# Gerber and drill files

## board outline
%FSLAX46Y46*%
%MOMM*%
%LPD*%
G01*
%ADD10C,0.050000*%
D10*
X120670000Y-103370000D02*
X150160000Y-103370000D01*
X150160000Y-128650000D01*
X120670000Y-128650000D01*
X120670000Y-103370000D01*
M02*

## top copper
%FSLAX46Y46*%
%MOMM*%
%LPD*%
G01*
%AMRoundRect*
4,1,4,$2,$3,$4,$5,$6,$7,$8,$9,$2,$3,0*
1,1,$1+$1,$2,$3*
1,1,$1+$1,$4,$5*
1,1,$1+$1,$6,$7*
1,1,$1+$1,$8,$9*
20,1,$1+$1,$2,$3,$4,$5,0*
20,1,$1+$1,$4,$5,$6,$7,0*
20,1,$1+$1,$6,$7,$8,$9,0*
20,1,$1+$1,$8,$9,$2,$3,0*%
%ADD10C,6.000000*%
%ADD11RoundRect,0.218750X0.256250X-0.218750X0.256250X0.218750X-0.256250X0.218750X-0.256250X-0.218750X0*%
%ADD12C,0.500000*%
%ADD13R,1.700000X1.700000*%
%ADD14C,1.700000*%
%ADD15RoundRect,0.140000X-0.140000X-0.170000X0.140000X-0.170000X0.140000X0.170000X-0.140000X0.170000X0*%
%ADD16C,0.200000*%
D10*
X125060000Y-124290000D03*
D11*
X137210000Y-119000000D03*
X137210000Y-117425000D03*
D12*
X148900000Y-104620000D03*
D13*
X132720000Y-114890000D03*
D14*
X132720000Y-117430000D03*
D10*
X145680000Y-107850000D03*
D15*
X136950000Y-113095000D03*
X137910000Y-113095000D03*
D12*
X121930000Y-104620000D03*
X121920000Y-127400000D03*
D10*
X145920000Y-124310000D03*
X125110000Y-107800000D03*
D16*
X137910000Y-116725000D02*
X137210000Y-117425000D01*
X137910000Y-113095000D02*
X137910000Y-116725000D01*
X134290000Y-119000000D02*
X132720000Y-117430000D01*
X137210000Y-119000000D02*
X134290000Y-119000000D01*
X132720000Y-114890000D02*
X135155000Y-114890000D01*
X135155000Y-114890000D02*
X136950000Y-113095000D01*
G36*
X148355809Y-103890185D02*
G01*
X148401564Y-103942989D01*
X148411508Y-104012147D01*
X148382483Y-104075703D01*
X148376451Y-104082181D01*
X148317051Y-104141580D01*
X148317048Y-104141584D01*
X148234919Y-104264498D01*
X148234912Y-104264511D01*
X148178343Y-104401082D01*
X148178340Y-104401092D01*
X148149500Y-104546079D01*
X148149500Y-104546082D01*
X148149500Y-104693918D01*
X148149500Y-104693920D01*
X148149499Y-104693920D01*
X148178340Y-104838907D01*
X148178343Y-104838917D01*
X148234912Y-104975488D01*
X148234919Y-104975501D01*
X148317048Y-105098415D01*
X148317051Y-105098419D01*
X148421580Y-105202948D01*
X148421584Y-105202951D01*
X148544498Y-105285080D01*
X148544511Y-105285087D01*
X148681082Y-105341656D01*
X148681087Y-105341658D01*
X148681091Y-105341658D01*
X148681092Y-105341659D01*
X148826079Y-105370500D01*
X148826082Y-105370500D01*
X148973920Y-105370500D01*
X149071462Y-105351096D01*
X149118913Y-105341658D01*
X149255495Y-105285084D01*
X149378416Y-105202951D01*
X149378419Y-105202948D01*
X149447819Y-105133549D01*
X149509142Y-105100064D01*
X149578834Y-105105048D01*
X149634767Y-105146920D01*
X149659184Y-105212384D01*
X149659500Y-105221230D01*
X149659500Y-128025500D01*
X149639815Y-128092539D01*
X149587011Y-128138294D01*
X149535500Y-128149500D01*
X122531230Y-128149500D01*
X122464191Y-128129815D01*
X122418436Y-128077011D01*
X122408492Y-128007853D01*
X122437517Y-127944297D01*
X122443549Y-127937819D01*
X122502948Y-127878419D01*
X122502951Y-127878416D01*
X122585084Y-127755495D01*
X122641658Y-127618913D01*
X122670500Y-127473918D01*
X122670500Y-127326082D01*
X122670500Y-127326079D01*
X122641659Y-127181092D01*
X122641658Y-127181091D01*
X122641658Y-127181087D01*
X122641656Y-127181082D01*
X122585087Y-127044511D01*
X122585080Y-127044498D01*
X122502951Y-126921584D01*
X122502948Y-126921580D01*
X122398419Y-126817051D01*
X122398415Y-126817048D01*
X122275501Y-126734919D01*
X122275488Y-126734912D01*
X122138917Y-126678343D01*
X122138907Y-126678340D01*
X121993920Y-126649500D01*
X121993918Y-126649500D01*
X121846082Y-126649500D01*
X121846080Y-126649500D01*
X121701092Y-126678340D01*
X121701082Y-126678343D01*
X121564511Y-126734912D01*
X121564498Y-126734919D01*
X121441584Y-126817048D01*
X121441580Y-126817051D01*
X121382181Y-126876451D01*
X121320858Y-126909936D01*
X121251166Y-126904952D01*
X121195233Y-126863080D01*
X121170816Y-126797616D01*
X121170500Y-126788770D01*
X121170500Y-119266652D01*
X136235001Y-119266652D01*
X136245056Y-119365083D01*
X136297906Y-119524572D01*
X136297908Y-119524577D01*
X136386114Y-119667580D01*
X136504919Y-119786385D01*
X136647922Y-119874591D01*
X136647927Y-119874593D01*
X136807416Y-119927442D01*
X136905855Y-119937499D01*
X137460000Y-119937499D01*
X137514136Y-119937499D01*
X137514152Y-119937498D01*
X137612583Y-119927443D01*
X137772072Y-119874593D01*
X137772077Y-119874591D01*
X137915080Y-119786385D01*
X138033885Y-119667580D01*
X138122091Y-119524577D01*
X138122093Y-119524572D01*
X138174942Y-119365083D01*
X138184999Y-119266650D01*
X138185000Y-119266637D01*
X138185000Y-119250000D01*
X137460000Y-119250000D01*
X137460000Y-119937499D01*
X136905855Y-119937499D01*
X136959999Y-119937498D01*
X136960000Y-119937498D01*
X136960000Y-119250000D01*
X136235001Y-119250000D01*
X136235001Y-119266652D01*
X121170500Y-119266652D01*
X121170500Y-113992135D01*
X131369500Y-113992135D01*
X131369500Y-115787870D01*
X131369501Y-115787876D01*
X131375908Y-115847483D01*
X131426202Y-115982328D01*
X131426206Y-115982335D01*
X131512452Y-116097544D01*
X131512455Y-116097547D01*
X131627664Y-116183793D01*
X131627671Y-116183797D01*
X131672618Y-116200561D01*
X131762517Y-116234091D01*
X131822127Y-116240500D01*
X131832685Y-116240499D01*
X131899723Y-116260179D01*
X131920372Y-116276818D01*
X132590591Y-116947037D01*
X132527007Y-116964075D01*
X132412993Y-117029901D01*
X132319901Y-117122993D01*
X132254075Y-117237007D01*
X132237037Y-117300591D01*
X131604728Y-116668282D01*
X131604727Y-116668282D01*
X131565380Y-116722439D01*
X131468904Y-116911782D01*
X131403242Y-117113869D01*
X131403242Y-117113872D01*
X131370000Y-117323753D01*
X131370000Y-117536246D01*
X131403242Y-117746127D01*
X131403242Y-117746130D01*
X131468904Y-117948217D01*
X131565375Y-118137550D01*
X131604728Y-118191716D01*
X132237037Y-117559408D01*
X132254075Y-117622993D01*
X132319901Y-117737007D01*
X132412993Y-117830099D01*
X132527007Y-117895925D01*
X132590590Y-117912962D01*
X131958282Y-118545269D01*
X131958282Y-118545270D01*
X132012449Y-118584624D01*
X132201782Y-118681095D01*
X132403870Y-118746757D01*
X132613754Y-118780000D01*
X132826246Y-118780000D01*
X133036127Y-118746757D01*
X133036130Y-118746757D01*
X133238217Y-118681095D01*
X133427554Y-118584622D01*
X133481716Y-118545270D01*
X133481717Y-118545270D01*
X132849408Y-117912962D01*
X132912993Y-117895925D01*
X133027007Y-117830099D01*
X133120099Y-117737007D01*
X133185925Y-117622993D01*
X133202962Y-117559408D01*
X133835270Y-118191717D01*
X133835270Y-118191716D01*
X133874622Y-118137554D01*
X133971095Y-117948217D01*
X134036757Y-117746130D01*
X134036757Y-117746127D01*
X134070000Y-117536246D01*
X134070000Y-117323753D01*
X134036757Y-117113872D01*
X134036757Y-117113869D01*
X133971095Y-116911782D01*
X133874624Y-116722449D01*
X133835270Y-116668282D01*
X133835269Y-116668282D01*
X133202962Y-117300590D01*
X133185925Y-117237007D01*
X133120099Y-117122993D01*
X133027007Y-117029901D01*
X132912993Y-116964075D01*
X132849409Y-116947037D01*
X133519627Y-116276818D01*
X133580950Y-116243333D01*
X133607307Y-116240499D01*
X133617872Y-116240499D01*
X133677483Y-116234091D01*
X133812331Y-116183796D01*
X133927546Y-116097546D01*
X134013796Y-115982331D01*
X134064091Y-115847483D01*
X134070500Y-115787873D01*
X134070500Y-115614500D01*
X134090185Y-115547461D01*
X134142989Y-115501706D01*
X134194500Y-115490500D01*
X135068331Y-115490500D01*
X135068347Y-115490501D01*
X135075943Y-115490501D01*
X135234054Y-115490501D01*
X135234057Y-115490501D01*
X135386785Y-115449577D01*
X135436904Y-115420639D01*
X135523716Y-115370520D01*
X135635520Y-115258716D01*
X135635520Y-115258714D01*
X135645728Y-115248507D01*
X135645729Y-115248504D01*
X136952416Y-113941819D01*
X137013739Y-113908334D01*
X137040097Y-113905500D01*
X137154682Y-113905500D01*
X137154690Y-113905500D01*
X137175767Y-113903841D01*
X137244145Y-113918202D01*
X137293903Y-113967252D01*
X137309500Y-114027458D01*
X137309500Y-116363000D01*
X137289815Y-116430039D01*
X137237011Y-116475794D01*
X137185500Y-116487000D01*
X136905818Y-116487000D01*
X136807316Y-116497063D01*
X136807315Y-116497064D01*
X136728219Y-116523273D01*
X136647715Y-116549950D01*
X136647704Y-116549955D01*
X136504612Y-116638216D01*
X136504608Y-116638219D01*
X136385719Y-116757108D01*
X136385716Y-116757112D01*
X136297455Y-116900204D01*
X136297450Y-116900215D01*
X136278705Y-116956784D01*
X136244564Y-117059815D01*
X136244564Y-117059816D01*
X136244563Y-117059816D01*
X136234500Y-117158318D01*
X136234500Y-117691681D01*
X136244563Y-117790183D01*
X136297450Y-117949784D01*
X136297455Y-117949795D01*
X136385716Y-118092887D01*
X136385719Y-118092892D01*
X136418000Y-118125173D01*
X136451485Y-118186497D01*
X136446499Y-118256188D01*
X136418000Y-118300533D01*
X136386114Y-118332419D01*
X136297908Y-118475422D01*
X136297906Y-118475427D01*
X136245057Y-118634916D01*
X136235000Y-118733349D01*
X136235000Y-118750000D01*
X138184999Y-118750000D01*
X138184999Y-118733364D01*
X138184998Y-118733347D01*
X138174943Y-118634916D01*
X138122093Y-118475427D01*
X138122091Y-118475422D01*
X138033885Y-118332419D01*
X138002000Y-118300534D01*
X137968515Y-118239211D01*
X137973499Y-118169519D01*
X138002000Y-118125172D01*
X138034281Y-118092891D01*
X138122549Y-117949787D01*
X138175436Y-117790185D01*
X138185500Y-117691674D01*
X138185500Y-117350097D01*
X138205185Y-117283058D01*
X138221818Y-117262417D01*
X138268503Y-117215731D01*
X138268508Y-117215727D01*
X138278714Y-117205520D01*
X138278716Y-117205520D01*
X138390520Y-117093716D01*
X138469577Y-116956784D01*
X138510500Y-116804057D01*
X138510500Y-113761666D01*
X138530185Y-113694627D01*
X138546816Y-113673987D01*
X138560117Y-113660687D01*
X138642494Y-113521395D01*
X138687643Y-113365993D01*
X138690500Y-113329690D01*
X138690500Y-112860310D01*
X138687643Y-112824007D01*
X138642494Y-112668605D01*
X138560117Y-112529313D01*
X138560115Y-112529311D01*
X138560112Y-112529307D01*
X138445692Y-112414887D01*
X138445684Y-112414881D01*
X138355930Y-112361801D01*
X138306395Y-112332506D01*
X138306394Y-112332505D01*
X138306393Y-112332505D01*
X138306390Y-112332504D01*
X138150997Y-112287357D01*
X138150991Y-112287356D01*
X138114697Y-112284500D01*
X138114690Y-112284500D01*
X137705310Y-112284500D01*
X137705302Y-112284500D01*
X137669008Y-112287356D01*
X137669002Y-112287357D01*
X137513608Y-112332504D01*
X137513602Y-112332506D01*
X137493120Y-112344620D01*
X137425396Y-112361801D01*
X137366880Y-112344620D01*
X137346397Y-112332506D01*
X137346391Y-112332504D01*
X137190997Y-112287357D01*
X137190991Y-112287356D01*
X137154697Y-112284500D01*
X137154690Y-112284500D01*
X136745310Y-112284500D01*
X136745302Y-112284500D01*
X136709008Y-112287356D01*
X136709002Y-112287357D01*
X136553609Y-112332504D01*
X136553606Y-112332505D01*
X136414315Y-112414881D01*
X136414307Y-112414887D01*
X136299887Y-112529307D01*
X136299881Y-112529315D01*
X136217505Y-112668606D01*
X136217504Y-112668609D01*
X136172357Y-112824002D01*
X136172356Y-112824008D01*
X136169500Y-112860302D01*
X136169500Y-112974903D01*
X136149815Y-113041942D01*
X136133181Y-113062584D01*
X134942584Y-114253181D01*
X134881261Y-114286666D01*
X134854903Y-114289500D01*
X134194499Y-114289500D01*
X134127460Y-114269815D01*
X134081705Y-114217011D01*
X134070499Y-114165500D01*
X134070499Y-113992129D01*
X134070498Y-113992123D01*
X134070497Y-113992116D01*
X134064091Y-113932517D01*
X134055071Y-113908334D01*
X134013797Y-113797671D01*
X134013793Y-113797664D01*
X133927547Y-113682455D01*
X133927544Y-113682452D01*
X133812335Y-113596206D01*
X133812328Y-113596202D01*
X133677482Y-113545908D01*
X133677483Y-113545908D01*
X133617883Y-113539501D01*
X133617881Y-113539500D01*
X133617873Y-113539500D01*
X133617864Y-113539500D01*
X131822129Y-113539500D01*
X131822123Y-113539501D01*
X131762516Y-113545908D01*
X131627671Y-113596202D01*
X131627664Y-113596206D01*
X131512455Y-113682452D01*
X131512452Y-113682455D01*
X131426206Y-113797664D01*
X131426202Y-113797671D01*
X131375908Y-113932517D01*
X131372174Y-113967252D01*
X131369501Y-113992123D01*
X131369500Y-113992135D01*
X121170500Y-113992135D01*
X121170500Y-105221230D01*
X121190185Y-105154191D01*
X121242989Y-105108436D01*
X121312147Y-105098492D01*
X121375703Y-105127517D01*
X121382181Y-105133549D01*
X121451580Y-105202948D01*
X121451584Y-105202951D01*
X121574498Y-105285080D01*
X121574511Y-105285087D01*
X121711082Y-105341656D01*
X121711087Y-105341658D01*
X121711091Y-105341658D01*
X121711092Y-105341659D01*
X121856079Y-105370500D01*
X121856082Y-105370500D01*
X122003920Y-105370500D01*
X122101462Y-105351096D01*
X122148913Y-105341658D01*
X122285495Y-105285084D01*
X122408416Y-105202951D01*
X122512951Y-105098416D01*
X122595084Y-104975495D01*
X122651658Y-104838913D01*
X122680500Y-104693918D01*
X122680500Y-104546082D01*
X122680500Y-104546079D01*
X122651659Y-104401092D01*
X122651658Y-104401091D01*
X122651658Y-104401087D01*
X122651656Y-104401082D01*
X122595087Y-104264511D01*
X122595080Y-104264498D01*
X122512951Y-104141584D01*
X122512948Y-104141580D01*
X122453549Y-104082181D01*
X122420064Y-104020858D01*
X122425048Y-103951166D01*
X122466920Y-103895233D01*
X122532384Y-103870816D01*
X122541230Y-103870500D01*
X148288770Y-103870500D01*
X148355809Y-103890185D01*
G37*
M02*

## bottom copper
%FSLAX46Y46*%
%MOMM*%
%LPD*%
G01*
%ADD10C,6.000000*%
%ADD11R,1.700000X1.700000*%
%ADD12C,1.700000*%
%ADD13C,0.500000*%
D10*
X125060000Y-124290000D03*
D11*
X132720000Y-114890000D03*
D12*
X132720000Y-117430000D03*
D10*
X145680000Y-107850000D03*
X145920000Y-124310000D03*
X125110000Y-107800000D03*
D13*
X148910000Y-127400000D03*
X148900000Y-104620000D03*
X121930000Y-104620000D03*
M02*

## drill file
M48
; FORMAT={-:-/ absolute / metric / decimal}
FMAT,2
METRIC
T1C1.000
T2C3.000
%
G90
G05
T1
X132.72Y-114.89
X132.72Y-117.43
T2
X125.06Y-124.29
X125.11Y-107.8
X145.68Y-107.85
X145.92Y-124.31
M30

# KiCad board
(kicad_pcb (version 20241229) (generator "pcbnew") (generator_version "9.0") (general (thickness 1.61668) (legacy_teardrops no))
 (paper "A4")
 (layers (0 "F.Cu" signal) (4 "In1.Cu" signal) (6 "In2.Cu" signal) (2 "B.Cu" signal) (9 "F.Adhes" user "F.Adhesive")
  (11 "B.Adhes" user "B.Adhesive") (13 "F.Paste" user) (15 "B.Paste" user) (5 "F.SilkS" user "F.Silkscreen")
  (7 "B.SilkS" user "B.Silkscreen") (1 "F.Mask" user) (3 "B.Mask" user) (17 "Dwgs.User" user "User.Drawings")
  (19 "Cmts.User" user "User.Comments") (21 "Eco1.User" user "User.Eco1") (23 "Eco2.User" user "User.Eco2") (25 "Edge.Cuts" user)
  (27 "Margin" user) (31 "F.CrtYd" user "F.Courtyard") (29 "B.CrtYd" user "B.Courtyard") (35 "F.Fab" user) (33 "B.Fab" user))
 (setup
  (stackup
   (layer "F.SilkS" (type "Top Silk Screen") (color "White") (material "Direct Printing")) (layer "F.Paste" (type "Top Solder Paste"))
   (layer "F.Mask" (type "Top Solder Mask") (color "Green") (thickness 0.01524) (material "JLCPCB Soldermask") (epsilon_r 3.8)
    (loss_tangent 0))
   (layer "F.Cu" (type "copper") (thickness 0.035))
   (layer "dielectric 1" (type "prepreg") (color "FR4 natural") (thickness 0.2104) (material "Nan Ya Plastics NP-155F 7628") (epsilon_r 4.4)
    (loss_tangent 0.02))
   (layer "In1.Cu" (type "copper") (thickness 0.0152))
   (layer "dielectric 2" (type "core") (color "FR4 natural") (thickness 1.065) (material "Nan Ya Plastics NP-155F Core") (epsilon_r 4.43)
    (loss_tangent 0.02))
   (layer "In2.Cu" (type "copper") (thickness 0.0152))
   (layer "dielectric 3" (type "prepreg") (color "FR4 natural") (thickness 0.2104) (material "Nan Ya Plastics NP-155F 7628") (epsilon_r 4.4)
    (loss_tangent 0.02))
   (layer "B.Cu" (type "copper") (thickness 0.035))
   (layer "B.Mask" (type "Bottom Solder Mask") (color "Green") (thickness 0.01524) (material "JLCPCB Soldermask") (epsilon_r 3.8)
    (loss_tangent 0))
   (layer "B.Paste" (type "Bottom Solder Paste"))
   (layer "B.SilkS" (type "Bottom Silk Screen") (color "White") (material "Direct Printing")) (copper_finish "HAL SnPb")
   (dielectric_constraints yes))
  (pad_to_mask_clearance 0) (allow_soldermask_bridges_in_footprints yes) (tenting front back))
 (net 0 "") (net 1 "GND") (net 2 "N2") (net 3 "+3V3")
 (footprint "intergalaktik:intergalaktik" (layer "F.Cu") (at 135.4 104.33)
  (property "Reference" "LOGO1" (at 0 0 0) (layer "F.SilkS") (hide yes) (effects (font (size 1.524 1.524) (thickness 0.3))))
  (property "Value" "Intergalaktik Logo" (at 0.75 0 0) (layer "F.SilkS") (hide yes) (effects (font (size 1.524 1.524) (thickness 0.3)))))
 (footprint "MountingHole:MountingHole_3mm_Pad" (layer "F.Cu") (at 125.06 124.29)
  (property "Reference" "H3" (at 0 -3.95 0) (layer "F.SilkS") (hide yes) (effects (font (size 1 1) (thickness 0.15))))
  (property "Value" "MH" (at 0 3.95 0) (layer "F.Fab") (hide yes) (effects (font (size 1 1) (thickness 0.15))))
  (pad "1" thru_hole circle (at 0 0) (size 6 6) (drill 3) (layers "*.Cu" "*.Mask") (remove_unused_layers no) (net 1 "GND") (zone_connect 2)))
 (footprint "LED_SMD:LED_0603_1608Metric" (layer "F.Cu") (at 137.21 118.2125 90)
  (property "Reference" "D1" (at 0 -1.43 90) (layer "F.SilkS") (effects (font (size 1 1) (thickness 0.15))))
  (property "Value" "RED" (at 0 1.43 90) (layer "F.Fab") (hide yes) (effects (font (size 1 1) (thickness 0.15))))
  (pad "1" smd roundrect (at -0.7875 0 90) (size 0.875 0.95) (layers "F.Cu" "F.Mask" "F.Paste") (roundrect_rratio 0.25) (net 1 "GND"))
  (pad "2" smd roundrect (at 0.7875 0 90) (size 0.875 0.95) (layers "F.Cu" "F.Mask" "F.Paste") (roundrect_rratio 0.25) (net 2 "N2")))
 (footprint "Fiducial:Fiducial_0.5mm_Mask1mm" (layer "F.Cu") (at 148.9 104.62)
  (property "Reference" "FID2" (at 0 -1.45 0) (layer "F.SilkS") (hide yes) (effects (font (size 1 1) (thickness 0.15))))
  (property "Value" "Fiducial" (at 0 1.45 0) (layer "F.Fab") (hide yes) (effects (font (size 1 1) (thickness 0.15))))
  (pad "" smd circle (at 0 0) (size 0.5 0.5) (layers "F.Cu" "F.Mask") (solder_mask_margin 0.25)))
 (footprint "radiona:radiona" (layer "F.Cu") (at 135.68 125.26)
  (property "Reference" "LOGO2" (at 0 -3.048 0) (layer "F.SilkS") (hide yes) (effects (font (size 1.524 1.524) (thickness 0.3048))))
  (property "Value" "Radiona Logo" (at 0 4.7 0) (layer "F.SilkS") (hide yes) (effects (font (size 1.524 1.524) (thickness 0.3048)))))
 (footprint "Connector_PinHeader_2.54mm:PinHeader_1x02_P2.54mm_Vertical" (layer "F.Cu") (at 132.72 114.89)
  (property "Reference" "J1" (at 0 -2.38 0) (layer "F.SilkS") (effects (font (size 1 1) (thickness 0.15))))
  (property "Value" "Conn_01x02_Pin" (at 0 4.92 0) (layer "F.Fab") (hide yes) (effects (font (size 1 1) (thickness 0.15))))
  (pad "1" thru_hole rect (at 0 0) (size 1.7 1.7) (drill 1) (layers "*.Cu" "*.Mask") (remove_unused_layers no) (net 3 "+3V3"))
  (pad "2" thru_hole circle (at 0 2.54) (size 1.7 1.7) (drill 1) (layers "*.Cu" "*.Mask") (remove_unused_layers no) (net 1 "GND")))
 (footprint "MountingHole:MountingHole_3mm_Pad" (layer "F.Cu") (at 145.68 107.85)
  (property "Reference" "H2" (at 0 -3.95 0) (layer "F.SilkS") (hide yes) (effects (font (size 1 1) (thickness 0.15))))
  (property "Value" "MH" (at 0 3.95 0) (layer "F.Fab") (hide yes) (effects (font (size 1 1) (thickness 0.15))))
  (pad "1" thru_hole circle (at 0 0) (size 6 6) (drill 3) (layers "*.Cu" "*.Mask") (remove_unused_layers no) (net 1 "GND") (zone_connect 2)))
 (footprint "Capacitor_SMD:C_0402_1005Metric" (layer "F.Cu") (at 137.43 113.095)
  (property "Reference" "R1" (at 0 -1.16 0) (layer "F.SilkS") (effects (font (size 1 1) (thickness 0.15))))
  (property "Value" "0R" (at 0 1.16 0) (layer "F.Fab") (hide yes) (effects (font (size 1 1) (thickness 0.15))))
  (pad "1" smd roundrect (at -0.48 0) (size 0.56 0.62) (layers "F.Cu" "F.Mask" "F.Paste") (roundrect_rratio 0.25) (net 3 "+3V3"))
  (pad "2" smd roundrect (at 0.48 0) (size 0.56 0.62) (layers "F.Cu" "F.Mask" "F.Paste") (roundrect_rratio 0.25) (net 2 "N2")))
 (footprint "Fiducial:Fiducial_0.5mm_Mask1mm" (layer "F.Cu") (at 121.93 104.62)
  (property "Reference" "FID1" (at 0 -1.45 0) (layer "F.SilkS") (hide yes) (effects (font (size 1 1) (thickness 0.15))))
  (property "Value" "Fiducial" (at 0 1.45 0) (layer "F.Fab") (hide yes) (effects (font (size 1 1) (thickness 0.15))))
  (pad "" smd circle (at 0 0) (size 0.5 0.5) (layers "F.Cu" "F.Mask") (solder_mask_margin 0.25)))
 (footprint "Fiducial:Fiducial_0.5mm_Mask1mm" (layer "F.Cu") (at 121.92 127.4)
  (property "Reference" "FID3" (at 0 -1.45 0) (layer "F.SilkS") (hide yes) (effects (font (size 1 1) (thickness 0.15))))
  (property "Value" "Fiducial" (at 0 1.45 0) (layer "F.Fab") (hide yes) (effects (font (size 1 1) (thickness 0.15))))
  (pad "" smd circle (at 0 0) (size 0.5 0.5) (layers "F.Cu" "F.Mask") (solder_mask_margin 0.25)))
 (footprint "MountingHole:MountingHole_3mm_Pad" (layer "F.Cu") (at 145.92 124.31)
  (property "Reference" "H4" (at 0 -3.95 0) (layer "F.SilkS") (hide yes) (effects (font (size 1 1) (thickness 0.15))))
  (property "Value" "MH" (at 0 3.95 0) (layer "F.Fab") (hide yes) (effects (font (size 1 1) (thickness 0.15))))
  (pad "1" thru_hole circle (at 0 0) (size 6 6) (drill 3) (layers "*.Cu" "*.Mask") (remove_unused_layers no) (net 1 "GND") (zone_connect 2)))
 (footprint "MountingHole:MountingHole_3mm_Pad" (layer "F.Cu") (at 125.11 107.8)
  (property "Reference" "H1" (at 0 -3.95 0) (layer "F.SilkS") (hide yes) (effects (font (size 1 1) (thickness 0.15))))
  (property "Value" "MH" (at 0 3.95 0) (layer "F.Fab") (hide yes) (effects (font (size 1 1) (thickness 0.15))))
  (pad "1" thru_hole circle (at 0 0) (size 6 6) (drill 3) (layers "*.Cu" "*.Mask") (remove_unused_layers no) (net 1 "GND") (zone_connect 2)))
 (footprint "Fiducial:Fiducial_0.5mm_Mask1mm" (layer "B.Cu") (at 148.91 127.4)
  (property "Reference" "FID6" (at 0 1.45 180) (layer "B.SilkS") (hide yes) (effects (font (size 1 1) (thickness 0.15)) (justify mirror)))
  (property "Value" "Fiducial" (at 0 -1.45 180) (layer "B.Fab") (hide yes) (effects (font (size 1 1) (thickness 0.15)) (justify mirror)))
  (pad "" smd circle (at 0 0) (size 0.5 0.5) (layers "B.Cu" "B.Mask") (solder_mask_margin 0.25)))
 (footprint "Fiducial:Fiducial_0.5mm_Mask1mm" (layer "B.Cu") (at 148.9 104.62)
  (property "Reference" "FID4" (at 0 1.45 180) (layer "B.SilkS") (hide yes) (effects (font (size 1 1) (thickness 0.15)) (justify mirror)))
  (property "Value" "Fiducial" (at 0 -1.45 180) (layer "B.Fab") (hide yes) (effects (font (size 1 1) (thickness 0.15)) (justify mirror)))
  (pad "" smd circle (at 0 0) (size 0.5 0.5) (layers "B.Cu" "B.Mask") (solder_mask_margin 0.25)))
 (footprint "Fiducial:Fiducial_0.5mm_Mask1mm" (layer "B.Cu") (at 121.93 104.62)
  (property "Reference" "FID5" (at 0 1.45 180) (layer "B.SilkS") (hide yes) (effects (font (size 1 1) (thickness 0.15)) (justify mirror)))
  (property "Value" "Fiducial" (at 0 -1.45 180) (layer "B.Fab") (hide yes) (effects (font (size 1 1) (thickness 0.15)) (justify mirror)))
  (pad "" smd circle (at 0 0) (size 0.5 0.5) (layers "B.Cu" "B.Mask") (solder_mask_margin 0.25)))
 (gr_rect (start 120.67 103.37) (end 150.16 128.65) (stroke (width 0.05) (type default)) (fill no) (layer "Edge.Cuts"))
 (segment (start 137.91 116.725) (end 137.21 117.425) (width 0.2) (layer "F.Cu") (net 2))
 (segment (start 137.91 113.095) (end 137.91 116.725) (width 0.2) (layer "F.Cu") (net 2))
 (segment (start 134.29 119) (end 132.72 117.43) (width 0.2) (layer "F.Cu") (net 1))
 (segment (start 137.21 119) (end 134.29 119) (width 0.2) (layer "F.Cu") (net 1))
 (segment (start 132.72 114.89) (end 135.155 114.89) (width 0.2) (layer "F.Cu") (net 3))
 (segment (start 135.155 114.89) (end 136.95 113.095) (width 0.2) (layer "F.Cu") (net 3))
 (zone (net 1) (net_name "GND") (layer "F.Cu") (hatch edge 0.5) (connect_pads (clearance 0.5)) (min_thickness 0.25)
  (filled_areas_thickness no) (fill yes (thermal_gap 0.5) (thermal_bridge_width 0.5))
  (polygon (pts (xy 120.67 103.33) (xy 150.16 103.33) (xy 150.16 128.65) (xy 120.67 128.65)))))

